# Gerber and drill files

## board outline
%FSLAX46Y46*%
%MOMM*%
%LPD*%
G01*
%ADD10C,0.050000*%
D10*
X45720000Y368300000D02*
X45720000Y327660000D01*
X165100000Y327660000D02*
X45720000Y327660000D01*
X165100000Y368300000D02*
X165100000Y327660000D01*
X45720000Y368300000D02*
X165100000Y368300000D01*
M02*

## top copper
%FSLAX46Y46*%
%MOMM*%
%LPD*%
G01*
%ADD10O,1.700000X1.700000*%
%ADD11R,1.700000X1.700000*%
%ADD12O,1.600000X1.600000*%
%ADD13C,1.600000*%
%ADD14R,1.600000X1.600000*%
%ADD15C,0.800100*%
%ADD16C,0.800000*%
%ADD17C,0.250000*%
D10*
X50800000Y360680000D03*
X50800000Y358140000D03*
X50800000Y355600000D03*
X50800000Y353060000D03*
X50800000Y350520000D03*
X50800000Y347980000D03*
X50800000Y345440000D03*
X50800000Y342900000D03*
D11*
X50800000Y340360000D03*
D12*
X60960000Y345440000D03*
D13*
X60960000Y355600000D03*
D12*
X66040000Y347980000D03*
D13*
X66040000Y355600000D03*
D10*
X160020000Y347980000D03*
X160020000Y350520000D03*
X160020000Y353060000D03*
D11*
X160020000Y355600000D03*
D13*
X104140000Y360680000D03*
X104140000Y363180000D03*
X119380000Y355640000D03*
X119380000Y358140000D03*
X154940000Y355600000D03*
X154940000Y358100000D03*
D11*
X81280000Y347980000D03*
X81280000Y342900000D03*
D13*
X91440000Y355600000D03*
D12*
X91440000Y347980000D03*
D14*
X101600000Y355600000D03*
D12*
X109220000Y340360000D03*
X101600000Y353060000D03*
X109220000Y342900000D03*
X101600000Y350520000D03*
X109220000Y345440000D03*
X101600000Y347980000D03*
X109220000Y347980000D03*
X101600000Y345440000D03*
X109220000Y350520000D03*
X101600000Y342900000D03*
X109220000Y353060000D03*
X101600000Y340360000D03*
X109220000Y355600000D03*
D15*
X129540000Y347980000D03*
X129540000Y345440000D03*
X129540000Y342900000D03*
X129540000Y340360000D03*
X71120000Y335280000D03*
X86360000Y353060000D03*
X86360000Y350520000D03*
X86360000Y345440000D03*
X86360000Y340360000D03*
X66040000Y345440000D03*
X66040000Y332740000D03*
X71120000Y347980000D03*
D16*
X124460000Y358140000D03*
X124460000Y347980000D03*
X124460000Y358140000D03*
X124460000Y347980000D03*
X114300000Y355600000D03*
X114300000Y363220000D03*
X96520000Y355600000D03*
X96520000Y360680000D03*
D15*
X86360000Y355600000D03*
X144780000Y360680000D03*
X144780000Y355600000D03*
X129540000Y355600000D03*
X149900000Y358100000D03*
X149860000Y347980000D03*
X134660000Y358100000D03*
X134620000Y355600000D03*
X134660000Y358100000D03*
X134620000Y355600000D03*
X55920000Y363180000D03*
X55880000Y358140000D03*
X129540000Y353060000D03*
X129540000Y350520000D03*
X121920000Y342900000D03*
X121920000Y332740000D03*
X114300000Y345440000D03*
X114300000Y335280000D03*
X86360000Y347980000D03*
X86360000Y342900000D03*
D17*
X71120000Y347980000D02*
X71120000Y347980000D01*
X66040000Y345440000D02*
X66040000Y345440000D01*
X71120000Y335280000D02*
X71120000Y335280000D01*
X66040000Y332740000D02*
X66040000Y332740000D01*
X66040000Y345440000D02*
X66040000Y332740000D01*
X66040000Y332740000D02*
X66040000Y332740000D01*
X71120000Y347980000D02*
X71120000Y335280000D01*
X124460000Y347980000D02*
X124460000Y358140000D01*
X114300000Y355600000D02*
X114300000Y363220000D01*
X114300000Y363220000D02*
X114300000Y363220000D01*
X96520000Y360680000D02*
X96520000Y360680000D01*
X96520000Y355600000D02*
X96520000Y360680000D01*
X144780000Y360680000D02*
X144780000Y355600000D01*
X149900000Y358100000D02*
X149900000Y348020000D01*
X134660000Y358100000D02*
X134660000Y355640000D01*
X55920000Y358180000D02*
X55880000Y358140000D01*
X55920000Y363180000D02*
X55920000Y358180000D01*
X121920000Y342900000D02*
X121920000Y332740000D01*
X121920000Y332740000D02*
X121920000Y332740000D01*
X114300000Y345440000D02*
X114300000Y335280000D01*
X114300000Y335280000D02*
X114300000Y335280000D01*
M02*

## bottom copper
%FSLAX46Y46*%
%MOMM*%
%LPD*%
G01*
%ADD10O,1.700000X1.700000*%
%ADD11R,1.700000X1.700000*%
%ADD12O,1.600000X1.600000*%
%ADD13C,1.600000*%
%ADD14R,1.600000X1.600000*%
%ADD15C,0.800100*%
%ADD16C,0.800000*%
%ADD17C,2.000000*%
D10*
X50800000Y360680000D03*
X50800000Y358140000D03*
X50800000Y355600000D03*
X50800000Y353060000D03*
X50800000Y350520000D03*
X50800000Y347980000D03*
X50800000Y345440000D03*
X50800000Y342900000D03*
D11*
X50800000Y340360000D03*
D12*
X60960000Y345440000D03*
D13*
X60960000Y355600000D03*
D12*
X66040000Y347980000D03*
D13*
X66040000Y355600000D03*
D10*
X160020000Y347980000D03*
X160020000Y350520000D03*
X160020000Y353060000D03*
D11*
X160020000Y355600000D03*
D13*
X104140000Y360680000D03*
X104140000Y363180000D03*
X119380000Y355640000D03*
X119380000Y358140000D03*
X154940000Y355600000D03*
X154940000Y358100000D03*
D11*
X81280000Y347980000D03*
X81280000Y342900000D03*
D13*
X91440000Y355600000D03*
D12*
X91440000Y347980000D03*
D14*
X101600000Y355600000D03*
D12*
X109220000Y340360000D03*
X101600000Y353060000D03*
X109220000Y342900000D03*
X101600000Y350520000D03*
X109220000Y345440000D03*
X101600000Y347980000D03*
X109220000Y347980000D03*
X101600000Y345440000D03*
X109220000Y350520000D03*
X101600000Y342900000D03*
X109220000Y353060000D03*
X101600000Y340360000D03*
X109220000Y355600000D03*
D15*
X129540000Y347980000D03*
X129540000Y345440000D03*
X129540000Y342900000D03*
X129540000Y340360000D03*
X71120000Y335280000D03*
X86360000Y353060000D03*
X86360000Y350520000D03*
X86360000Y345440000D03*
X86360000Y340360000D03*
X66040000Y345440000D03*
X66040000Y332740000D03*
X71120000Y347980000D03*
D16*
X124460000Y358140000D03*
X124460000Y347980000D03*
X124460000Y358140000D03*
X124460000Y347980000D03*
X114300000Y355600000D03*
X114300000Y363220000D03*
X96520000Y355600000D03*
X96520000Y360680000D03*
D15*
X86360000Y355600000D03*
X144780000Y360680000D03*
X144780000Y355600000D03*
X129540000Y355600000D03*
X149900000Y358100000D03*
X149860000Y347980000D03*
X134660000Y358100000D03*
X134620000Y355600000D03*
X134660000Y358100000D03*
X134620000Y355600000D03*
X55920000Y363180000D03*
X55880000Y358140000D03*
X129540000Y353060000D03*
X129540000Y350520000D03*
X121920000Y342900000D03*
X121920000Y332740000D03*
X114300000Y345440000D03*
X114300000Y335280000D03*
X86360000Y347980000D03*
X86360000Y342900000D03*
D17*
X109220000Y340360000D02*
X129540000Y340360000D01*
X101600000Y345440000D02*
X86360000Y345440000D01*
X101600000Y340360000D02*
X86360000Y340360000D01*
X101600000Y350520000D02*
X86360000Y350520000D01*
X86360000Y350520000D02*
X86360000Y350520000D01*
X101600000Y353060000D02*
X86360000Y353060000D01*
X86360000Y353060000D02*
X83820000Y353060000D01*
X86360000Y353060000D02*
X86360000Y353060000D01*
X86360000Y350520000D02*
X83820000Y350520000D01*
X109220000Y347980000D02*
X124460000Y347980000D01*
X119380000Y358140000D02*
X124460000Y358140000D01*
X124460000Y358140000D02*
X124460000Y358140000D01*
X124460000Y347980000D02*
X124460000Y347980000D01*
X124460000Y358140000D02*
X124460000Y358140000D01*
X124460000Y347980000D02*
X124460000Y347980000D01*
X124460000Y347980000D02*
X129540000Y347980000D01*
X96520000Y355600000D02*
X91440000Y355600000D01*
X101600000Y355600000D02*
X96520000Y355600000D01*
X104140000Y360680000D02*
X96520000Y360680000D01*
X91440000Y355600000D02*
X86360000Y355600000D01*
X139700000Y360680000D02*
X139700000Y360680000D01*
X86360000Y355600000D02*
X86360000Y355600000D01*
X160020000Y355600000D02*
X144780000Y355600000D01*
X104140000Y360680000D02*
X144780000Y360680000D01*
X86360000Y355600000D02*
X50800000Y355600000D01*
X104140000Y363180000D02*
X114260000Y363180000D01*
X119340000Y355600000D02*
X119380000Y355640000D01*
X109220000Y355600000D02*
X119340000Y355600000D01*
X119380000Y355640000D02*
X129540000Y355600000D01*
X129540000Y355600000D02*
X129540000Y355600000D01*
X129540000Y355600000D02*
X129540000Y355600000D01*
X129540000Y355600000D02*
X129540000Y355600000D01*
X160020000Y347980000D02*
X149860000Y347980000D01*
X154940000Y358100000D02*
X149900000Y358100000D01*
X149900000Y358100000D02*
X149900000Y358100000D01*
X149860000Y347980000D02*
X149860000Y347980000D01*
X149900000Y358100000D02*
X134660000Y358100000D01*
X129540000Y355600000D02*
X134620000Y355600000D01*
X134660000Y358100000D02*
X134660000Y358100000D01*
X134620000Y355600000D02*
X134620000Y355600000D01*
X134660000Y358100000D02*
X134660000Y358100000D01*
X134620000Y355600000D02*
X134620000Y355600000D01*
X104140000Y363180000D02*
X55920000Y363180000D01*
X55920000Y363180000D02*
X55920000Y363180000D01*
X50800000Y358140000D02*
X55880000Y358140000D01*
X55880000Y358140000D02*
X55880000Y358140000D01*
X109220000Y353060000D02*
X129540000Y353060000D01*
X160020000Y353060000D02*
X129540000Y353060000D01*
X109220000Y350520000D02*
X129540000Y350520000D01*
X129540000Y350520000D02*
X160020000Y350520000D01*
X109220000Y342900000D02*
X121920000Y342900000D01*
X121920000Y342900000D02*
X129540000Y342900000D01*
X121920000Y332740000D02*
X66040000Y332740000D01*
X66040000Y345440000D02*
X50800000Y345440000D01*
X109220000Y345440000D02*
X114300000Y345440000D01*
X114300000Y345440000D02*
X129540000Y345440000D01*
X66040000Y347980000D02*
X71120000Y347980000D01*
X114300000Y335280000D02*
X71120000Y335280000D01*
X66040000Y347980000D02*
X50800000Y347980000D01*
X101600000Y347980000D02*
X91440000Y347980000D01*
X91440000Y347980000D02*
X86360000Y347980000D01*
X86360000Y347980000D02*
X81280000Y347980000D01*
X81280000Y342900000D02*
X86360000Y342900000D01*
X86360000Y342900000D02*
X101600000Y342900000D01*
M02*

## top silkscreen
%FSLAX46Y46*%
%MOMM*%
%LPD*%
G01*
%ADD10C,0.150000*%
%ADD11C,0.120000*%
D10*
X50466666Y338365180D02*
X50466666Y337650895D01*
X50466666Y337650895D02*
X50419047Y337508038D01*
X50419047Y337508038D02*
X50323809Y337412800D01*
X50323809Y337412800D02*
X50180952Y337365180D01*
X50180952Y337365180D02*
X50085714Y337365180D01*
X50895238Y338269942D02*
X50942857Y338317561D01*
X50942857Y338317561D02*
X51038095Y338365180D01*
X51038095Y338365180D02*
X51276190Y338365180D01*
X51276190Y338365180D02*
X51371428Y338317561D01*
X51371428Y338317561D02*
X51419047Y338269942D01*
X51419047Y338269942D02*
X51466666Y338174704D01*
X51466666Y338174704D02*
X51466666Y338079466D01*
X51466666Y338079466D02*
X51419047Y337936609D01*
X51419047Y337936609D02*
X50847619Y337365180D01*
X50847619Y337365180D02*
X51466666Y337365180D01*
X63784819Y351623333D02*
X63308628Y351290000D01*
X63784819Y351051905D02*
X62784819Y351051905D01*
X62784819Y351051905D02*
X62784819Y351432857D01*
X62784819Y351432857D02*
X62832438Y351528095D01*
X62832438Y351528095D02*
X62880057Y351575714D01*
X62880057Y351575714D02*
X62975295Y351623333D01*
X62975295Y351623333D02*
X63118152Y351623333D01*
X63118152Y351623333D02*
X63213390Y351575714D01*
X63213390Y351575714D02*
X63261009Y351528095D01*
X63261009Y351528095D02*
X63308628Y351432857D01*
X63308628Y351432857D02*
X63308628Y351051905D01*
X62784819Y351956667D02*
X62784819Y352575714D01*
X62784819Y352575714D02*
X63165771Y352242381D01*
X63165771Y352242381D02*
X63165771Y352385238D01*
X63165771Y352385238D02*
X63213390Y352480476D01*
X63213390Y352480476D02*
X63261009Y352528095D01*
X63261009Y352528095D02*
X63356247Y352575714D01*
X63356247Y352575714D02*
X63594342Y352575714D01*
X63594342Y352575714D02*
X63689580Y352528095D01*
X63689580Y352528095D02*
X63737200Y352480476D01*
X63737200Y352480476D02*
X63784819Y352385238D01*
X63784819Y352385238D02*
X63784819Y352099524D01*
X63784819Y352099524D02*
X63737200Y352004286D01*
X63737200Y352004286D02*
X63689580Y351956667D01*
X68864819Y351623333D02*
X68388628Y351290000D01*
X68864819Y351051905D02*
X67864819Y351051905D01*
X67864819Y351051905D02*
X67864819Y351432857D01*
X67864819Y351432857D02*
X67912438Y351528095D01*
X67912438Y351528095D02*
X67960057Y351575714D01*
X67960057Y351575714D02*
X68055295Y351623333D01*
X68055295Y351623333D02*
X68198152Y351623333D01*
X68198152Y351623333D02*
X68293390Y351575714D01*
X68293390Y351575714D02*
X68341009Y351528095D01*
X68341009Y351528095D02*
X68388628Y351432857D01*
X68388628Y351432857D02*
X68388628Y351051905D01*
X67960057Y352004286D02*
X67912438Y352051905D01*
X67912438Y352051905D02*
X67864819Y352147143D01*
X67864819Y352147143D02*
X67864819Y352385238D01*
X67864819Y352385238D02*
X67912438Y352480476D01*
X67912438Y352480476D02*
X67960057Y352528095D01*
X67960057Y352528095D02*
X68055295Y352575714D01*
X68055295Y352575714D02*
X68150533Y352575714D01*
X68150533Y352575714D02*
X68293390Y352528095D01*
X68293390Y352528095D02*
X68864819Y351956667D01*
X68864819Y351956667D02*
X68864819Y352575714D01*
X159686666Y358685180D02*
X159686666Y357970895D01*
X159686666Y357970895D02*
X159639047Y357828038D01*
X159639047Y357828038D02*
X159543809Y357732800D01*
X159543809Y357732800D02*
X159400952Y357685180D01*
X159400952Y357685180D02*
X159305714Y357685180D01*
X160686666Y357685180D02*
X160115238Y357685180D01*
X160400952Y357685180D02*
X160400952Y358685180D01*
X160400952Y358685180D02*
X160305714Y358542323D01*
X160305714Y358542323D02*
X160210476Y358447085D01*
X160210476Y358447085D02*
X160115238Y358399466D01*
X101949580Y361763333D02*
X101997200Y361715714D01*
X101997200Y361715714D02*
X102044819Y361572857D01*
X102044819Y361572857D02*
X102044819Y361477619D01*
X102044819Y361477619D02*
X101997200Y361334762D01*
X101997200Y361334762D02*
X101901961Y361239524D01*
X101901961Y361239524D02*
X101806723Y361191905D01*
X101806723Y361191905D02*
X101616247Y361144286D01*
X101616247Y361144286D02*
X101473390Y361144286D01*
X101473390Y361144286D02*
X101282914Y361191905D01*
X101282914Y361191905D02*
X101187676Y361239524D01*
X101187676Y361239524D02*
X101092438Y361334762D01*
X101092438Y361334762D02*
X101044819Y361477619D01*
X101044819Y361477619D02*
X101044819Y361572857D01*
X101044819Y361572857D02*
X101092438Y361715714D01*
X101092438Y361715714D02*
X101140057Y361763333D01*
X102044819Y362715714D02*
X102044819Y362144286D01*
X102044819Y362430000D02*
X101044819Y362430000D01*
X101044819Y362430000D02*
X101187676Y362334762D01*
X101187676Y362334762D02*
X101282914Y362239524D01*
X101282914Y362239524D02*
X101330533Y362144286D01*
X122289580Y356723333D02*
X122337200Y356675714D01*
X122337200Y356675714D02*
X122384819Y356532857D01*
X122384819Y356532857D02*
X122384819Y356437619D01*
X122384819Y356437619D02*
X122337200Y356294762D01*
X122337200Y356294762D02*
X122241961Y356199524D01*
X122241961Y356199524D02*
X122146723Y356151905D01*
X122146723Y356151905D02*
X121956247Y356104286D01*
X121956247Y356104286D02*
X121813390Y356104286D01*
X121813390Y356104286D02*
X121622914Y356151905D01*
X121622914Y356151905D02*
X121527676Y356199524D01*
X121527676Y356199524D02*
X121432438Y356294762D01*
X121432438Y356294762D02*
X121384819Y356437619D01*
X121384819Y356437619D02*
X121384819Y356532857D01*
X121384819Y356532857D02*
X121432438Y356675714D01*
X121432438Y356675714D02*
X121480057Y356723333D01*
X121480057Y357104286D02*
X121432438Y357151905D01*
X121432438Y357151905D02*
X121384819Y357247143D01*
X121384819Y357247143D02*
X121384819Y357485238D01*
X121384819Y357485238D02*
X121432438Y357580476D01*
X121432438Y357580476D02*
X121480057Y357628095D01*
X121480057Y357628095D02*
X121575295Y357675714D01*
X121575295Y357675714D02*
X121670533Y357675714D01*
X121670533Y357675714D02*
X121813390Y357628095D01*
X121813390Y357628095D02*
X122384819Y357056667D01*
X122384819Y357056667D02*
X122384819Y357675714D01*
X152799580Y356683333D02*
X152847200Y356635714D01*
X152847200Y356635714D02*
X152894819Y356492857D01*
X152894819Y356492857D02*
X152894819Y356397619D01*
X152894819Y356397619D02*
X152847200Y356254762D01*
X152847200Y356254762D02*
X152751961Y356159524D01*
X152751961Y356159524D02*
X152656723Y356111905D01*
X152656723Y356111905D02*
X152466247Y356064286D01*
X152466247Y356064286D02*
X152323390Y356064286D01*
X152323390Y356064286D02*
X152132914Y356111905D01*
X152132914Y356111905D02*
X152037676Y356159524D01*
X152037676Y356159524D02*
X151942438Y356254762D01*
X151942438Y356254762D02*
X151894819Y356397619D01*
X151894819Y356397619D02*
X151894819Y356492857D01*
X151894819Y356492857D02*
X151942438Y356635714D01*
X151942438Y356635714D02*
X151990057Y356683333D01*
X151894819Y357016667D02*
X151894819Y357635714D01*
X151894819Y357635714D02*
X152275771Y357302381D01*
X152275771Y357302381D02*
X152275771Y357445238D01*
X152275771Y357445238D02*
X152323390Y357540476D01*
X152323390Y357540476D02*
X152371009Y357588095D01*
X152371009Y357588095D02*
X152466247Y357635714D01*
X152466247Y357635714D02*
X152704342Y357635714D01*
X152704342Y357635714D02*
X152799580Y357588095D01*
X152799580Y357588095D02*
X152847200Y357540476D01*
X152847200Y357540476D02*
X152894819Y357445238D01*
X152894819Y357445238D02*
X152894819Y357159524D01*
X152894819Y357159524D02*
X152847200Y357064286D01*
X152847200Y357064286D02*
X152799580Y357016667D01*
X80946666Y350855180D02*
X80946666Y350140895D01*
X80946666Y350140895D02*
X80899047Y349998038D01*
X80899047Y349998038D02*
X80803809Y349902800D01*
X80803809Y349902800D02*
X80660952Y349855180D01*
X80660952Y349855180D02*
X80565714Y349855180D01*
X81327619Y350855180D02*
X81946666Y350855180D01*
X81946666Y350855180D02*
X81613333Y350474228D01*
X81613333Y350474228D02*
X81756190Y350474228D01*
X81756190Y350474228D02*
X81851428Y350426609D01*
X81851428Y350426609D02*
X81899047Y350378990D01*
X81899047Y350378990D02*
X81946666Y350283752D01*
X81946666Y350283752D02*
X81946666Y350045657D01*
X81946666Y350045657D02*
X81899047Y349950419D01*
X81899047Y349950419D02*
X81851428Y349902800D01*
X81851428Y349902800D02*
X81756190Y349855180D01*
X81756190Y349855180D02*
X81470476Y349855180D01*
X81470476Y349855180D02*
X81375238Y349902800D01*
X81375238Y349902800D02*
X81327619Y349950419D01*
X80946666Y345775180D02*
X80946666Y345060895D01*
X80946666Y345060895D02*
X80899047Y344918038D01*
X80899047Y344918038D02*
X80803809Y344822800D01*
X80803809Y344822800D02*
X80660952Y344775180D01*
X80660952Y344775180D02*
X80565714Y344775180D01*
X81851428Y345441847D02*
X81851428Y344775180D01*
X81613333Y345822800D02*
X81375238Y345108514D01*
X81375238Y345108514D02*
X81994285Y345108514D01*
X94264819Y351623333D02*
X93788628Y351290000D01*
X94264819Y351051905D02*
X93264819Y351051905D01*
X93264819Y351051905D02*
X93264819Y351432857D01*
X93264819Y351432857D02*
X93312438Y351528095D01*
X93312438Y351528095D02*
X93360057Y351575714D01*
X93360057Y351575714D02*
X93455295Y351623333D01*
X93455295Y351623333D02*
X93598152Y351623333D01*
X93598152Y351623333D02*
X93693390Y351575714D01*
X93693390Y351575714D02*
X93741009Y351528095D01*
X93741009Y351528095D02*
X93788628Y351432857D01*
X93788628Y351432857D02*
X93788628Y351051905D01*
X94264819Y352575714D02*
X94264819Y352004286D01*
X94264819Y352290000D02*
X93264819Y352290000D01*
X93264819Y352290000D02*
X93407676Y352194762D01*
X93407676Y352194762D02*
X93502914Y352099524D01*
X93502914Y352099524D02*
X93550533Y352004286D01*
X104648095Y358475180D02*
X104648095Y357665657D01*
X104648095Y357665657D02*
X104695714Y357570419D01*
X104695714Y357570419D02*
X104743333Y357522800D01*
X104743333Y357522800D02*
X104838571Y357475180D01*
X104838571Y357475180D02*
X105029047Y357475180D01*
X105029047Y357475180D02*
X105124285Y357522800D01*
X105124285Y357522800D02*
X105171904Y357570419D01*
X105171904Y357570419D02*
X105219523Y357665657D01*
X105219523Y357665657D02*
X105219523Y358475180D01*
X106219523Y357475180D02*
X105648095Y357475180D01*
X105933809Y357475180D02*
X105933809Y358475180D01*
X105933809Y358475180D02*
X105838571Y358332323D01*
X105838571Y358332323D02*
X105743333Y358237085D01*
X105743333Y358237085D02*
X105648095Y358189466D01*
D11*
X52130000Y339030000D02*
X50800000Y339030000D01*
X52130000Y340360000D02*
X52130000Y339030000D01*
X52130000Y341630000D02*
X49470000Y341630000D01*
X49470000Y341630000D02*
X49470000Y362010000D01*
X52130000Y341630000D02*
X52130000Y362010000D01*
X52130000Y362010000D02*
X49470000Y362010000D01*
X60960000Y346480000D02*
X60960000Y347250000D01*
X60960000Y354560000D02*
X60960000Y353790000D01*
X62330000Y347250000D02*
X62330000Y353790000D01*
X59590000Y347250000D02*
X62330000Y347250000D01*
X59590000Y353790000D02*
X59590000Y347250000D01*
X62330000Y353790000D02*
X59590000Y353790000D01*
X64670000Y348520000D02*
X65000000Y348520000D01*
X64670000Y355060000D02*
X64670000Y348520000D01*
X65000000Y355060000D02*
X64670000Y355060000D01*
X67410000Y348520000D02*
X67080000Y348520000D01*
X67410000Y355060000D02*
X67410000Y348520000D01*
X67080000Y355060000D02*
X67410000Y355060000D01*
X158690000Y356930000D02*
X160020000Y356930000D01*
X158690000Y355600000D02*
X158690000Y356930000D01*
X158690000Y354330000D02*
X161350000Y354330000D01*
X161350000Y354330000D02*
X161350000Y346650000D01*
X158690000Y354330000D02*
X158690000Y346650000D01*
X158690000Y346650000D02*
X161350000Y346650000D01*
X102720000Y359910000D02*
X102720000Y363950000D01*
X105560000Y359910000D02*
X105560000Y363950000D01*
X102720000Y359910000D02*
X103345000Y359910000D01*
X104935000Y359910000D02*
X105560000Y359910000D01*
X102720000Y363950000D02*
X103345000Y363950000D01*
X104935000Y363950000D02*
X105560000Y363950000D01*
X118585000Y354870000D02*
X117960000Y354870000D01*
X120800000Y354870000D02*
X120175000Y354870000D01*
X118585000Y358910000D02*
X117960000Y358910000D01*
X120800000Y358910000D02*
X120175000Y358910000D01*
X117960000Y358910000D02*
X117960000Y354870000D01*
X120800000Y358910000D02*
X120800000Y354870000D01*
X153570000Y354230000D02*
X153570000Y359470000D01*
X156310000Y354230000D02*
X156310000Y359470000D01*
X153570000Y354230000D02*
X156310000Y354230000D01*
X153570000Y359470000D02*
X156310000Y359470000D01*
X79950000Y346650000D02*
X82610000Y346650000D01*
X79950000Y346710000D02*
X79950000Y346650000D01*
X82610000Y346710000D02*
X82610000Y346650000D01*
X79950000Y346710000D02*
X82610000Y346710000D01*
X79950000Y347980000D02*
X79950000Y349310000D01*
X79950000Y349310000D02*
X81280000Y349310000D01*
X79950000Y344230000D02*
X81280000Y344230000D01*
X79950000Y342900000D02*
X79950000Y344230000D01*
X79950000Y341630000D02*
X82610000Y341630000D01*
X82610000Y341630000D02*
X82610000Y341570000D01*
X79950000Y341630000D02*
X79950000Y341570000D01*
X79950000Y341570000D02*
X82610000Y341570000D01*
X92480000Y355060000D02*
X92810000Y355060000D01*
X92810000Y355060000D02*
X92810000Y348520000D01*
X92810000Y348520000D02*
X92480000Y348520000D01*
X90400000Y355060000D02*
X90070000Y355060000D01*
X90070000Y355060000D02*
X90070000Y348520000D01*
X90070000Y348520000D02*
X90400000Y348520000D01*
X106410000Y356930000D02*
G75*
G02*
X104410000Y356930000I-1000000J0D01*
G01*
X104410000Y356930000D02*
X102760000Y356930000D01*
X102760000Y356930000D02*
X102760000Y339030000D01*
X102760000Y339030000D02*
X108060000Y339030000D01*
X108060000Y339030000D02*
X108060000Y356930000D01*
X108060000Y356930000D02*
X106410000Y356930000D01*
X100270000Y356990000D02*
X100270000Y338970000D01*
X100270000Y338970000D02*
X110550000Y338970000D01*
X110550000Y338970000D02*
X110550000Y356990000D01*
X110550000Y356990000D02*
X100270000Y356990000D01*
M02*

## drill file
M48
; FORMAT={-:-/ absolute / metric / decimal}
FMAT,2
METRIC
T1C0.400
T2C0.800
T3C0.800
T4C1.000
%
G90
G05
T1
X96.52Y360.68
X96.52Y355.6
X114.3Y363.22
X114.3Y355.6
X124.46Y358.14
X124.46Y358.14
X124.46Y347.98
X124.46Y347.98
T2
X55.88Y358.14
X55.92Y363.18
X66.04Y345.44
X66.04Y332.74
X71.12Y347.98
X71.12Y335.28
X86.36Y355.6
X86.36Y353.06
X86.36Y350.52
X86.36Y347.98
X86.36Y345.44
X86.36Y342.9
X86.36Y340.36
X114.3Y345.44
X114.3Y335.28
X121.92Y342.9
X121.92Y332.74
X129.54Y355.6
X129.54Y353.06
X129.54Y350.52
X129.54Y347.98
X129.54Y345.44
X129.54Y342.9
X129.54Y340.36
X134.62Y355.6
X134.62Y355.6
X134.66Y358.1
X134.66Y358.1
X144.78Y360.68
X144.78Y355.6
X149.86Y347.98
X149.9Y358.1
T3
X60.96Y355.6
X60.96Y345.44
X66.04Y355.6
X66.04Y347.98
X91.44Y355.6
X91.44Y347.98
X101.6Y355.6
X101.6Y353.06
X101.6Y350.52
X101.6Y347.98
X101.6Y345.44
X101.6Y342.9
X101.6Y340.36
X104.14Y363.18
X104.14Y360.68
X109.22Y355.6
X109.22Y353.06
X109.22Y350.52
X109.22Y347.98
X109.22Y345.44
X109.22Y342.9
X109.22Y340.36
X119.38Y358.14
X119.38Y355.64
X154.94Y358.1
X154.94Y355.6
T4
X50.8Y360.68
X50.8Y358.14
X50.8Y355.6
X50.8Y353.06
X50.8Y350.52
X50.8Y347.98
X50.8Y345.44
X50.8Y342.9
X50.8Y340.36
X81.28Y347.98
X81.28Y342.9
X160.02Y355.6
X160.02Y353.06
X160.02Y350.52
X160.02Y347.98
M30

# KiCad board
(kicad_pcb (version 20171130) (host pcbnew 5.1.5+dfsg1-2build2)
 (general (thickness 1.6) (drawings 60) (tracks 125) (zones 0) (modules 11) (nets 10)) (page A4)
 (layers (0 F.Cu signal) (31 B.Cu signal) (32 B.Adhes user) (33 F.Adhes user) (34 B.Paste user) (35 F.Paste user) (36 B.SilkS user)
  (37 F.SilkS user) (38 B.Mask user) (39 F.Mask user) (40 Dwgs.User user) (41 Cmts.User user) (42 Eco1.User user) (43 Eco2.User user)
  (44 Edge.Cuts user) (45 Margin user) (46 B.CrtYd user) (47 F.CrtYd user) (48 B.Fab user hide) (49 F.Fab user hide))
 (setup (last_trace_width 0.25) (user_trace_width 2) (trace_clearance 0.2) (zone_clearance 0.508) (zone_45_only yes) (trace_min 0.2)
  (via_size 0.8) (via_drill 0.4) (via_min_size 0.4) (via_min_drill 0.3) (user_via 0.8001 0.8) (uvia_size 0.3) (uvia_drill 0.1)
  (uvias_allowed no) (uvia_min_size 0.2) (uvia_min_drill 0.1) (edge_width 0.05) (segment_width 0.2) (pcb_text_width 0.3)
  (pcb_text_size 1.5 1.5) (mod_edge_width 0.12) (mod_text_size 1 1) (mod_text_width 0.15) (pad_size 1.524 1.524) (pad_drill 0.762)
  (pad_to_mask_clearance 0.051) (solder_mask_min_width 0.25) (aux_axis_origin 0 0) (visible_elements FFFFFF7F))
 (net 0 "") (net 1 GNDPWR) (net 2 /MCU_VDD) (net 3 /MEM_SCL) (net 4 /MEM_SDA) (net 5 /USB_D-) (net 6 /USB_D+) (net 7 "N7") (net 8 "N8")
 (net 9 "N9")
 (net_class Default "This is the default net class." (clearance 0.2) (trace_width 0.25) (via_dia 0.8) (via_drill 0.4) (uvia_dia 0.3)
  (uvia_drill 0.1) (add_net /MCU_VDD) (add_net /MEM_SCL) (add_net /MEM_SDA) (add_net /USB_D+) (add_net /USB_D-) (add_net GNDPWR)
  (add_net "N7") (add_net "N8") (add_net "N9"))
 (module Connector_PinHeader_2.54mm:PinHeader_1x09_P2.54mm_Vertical (layer F.Cu) (at 50.8 -340.36 180)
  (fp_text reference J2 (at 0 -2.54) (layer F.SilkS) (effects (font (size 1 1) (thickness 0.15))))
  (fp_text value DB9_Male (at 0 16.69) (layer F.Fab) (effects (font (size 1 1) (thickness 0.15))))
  (fp_line (start -1.33 -1.33) (end 0 -1.33) (layer F.SilkS) (width 0.12))
  (fp_line (start -1.33 0) (end -1.33 -1.33) (layer F.SilkS) (width 0.12))
  (fp_line (start -1.33 1.27) (end 1.33 1.27) (layer F.SilkS) (width 0.12))
  (fp_line (start 1.33 1.27) (end 1.33 21.65) (layer F.SilkS) (width 0.12))
  (fp_line (start -1.33 1.27) (end -1.33 21.65) (layer F.SilkS) (width 0.12))
  (fp_line (start -1.33 21.65) (end 1.33 21.65) (layer F.SilkS) (width 0.12))
  (pad 9 thru_hole oval (at 0 20.32 180) (size 1.7 1.7) (drill 1) (layers *.Cu *.Mask))
  (pad 8 thru_hole oval (at 0 17.78 180) (size 1.7 1.7) (drill 1) (layers *.Cu *.Mask) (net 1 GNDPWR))
  (pad 7 thru_hole oval (at 0 15.24 180) (size 1.7 1.7) (drill 1) (layers *.Cu *.Mask) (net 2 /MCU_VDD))
  (pad 6 thru_hole oval (at 0 12.7 180) (size 1.7 1.7) (drill 1) (layers *.Cu *.Mask))
  (pad 5 thru_hole oval (at 0 10.16 180) (size 1.7 1.7) (drill 1) (layers *.Cu *.Mask))
  (pad 4 thru_hole oval (at 0 7.62 180) (size 1.7 1.7) (drill 1) (layers *.Cu *.Mask) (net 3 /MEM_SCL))
  (pad 3 thru_hole oval (at 0 5.08 180) (size 1.7 1.7) (drill 1) (layers *.Cu *.Mask) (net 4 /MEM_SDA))
  (pad 2 thru_hole oval (at 0 2.54 180) (size 1.7 1.7) (drill 1) (layers *.Cu *.Mask))
  (pad 1 thru_hole rect (at 0 0 180) (size 1.7 1.7) (drill 1) (layers *.Cu *.Mask)))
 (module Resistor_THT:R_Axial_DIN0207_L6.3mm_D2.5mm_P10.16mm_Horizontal (layer F.Cu) (at 60.96 -355.6 270)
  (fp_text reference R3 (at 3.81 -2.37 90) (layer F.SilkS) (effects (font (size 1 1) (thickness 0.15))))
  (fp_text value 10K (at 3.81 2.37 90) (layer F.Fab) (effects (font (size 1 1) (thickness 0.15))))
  (fp_line (start 9.12 0) (end 8.35 0) (layer F.SilkS) (width 0.12))
  (fp_line (start 1.04 0) (end 1.81 0) (layer F.SilkS) (width 0.12))
  (fp_line (start 8.35 -1.37) (end 1.81 -1.37) (layer F.SilkS) (width 0.12))
  (fp_line (start 8.35 1.37) (end 8.35 -1.37) (layer F.SilkS) (width 0.12))
  (fp_line (start 1.81 1.37) (end 8.35 1.37) (layer F.SilkS) (width 0.12))
  (fp_line (start 1.81 -1.37) (end 1.81 1.37) (layer F.SilkS) (width 0.12))
  (pad 2 thru_hole oval (at 10.16 0 270) (size 1.6 1.6) (drill 0.8) (layers *.Cu *.Mask) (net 4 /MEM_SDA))
  (pad 1 thru_hole circle (at 0 0 270) (size 1.6 1.6) (drill 0.8) (layers *.Cu *.Mask) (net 2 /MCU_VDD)))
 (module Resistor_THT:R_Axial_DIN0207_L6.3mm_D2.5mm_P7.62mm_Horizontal (layer F.Cu) (at 66.04 -355.6 270)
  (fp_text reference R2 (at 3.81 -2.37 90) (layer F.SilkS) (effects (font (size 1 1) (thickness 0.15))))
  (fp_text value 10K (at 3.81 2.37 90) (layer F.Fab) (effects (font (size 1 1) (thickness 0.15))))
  (fp_line (start 7.08 1.37) (end 7.08 1.04) (layer F.SilkS) (width 0.12))
  (fp_line (start 0.54 1.37) (end 7.08 1.37) (layer F.SilkS) (width 0.12))
  (fp_line (start 0.54 1.04) (end 0.54 1.37) (layer F.SilkS) (width 0.12))
  (fp_line (start 7.08 -1.37) (end 7.08 -1.04) (layer F.SilkS) (width 0.12))
  (fp_line (start 0.54 -1.37) (end 7.08 -1.37) (layer F.SilkS) (width 0.12))
  (fp_line (start 0.54 -1.04) (end 0.54 -1.37) (layer F.SilkS) (width 0.12))
  (pad 2 thru_hole oval (at 7.62 0 270) (size 1.6 1.6) (drill 0.8) (layers *.Cu *.Mask) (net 3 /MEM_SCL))
  (pad 1 thru_hole circle (at 0 0 270) (size 1.6 1.6) (drill 0.8) (layers *.Cu *.Mask) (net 2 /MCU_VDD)))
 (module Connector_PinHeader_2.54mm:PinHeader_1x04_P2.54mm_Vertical (layer F.Cu) (at 160.02 -355.6)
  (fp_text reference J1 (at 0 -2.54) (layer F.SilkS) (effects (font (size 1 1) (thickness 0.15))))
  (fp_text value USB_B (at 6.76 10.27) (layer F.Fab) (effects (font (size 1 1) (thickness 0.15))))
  (fp_line (start -1.33 -1.33) (end 0 -1.33) (layer F.SilkS) (width 0.12))
  (fp_line (start -1.33 0) (end -1.33 -1.33) (layer F.SilkS) (width 0.12))
  (fp_line (start -1.33 1.27) (end 1.33 1.27) (layer F.SilkS) (width 0.12))
  (fp_line (start 1.33 1.27) (end 1.33 8.95) (layer F.SilkS) (width 0.12))
  (fp_line (start -1.33 1.27) (end -1.33 8.95) (layer F.SilkS) (width 0.12))
  (fp_line (start -1.33 8.95) (end 1.33 8.95) (layer F.SilkS) (width 0.12))
  (pad 4 thru_hole oval (at 0 7.62) (size 1.7 1.7) (drill 1) (layers *.Cu *.Mask) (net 1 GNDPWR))
  (pad 3 thru_hole oval (at 0 5.08) (size 1.7 1.7) (drill 1) (layers *.Cu *.Mask) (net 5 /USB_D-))
  (pad 2 thru_hole oval (at 0 2.54) (size 1.7 1.7) (drill 1) (layers *.Cu *.Mask) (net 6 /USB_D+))
  (pad 1 thru_hole rect (at 0 0) (size 1.7 1.7) (drill 1) (layers *.Cu *.Mask) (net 2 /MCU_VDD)))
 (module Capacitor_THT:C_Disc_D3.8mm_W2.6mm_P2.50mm (layer F.Cu) (at 104.14 -360.68 90)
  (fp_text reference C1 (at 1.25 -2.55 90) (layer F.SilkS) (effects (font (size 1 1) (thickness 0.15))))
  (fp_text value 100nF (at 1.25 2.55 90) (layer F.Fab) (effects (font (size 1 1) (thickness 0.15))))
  (fp_line (start -0.77 -1.42) (end 3.27 -1.42) (layer F.SilkS) (width 0.12))
  (fp_line (start -0.77 1.42) (end 3.27 1.42) (layer F.SilkS) (width 0.12))
  (fp_line (start -0.77 -1.42) (end -0.77 -0.795) (layer F.SilkS) (width 0.12))
  (fp_line (start -0.77 0.795) (end -0.77 1.42) (layer F.SilkS) (width 0.12))
  (fp_line (start 3.27 -1.42) (end 3.27 -0.795) (layer F.SilkS) (width 0.12))
  (fp_line (start 3.27 0.795) (end 3.27 1.42) (layer F.SilkS) (width 0.12))
  (pad 1 thru_hole circle (at 0 0 90) (size 1.6 1.6) (drill 0.8) (layers *.Cu *.Mask) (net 2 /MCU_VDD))
  (pad 2 thru_hole circle (at 2.5 0 90) (size 1.6 1.6) (drill 0.8) (layers *.Cu *.Mask) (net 1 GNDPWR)))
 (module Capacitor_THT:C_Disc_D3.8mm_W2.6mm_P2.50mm (layer F.Cu) (at 119.38 -358.14 270)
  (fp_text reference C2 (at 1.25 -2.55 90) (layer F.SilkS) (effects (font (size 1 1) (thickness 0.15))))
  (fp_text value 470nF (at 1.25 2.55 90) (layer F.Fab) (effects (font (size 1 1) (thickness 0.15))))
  (fp_line (start 3.27 0.795) (end 3.27 1.42) (layer F.SilkS) (width 0.12))
  (fp_line (start 3.27 -1.42) (end 3.27 -0.795) (layer F.SilkS) (width 0.12))
  (fp_line (start -0.77 0.795) (end -0.77 1.42) (layer F.SilkS) (width 0.12))
  (fp_line (start -0.77 -1.42) (end -0.77 -0.795) (layer F.SilkS) (width 0.12))
  (fp_line (start -0.77 1.42) (end 3.27 1.42) (layer F.SilkS) (width 0.12))
  (fp_line (start -0.77 -1.42) (end 3.27 -1.42) (layer F.SilkS) (width 0.12))
  (pad 2 thru_hole circle (at 2.5 0 270) (size 1.6 1.6) (drill 0.8) (layers *.Cu *.Mask) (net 1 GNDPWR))
  (pad 1 thru_hole circle (at 0 0 270) (size 1.6 1.6) (drill 0.8) (layers *.Cu *.Mask) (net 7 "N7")))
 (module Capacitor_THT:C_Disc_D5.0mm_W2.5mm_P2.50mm (layer F.Cu) (at 154.94 -355.6 90)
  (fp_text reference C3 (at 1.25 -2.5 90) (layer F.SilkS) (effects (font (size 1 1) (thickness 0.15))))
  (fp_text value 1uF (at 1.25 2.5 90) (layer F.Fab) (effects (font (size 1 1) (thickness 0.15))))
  (fp_line (start -1.37 -1.37) (end 3.87 -1.37) (layer F.SilkS) (width 0.12))
  (fp_line (start -1.37 1.37) (end 3.87 1.37) (layer F.SilkS) (width 0.12))
  (fp_line (start -1.37 -1.37) (end -1.37 1.37) (layer F.SilkS) (width 0.12))
  (fp_line (start 3.87 -1.37) (end 3.87 1.37) (layer F.SilkS) (width 0.12))
  (pad 1 thru_hole circle (at 0 0 90) (size 1.6 1.6) (drill 0.8) (layers *.Cu *.Mask) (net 2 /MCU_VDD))
  (pad 2 thru_hole circle (at 2.5 0 90) (size 1.6 1.6) (drill 0.8) (layers *.Cu *.Mask) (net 1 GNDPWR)))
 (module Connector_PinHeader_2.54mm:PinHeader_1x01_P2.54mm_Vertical (layer F.Cu) (at 81.28 -347.98)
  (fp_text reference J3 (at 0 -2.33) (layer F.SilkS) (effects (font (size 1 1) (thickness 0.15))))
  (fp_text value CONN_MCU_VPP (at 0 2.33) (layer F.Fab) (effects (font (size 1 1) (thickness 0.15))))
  (fp_line (start -1.33 1.33) (end 1.33 1.33) (layer F.SilkS) (width 0.12))
  (fp_line (start -1.33 1.27) (end -1.33 1.33) (layer F.SilkS) (width 0.12))
  (fp_line (start 1.33 1.27) (end 1.33 1.33) (layer F.SilkS) (width 0.12))
  (fp_line (start -1.33 1.27) (end 1.33 1.27) (layer F.SilkS) (width 0.12))
  (fp_line (start -1.33 0) (end -1.33 -1.33) (layer F.SilkS) (width 0.12))
  (fp_line (start -1.33 -1.33) (end 0 -1.33) (layer F.SilkS) (width 0.12))
  (pad 1 thru_hole rect (at 0 0) (size 1.7 1.7) (drill 1) (layers *.Cu *.Mask) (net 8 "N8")))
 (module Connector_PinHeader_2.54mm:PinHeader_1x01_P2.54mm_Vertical (layer F.Cu) (at 81.28 -342.9)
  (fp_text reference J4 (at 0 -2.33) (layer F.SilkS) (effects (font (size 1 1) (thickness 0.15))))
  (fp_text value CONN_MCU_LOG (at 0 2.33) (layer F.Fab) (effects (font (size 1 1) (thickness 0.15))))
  (fp_line (start -1.33 -1.33) (end 0 -1.33) (layer F.SilkS) (width 0.12))
  (fp_line (start -1.33 0) (end -1.33 -1.33) (layer F.SilkS) (width 0.12))
  (fp_line (start -1.33 1.27) (end 1.33 1.27) (layer F.SilkS) (width 0.12))
  (fp_line (start 1.33 1.27) (end 1.33 1.33) (layer F.SilkS) (width 0.12))
  (fp_line (start -1.33 1.27) (end -1.33 1.33) (layer F.SilkS) (width 0.12))
  (fp_line (start -1.33 1.33) (end 1.33 1.33) (layer F.SilkS) (width 0.12))
  (pad 1 thru_hole rect (at 0 0) (size 1.7 1.7) (drill 1) (layers *.Cu *.Mask) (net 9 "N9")))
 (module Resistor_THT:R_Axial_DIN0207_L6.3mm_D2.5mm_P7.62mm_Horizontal (layer F.Cu) (at 91.44 -355.6 270)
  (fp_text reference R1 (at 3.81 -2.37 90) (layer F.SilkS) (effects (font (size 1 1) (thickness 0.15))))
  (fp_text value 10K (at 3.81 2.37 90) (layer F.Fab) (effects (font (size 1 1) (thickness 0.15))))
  (fp_line (start 0.54 -1.04) (end 0.54 -1.37) (layer F.SilkS) (width 0.12))
  (fp_line (start 0.54 -1.37) (end 7.08 -1.37) (layer F.SilkS) (width 0.12))
  (fp_line (start 7.08 -1.37) (end 7.08 -1.04) (layer F.SilkS) (width 0.12))
  (fp_line (start 0.54 1.04) (end 0.54 1.37) (layer F.SilkS) (width 0.12))
  (fp_line (start 0.54 1.37) (end 7.08 1.37) (layer F.SilkS) (width 0.12))
  (fp_line (start 7.08 1.37) (end 7.08 1.04) (layer F.SilkS) (width 0.12))
  (pad 1 thru_hole circle (at 0 0 270) (size 1.6 1.6) (drill 0.8) (layers *.Cu *.Mask) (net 2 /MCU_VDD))
  (pad 2 thru_hole oval (at 7.62 0 270) (size 1.6 1.6) (drill 0.8) (layers *.Cu *.Mask) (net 8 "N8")))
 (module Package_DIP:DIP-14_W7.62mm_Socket (layer F.Cu) (at 101.6 -355.6)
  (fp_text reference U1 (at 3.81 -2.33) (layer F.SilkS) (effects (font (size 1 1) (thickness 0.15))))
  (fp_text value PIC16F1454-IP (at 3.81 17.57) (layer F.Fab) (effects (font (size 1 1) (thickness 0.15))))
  (fp_arc (start 3.81 -1.33) (end 2.81 -1.33) (angle -180) (layer F.SilkS) (width 0.12))
  (fp_line (start 2.81 -1.33) (end 1.16 -1.33) (layer F.SilkS) (width 0.12))
  (fp_line (start 1.16 -1.33) (end 1.16 16.57) (layer F.SilkS) (width 0.12))
  (fp_line (start 1.16 16.57) (end 6.46 16.57) (layer F.SilkS) (width 0.12))
  (fp_line (start 6.46 16.57) (end 6.46 -1.33) (layer F.SilkS) (width 0.12))
  (fp_line (start 6.46 -1.33) (end 4.81 -1.33) (layer F.SilkS) (width 0.12))
  (fp_line (start -1.33 -1.39) (end -1.33 16.63) (layer F.SilkS) (width 0.12))
  (fp_line (start -1.33 16.63) (end 8.95 16.63) (layer F.SilkS) (width 0.12))
  (fp_line (start 8.95 16.63) (end 8.95 -1.39) (layer F.SilkS) (width 0.12))
  (fp_line (start 8.95 -1.39) (end -1.33 -1.39) (layer F.SilkS) (width 0.12))
  (pad 1 thru_hole rect (at 0 0) (size 1.6 1.6) (drill 0.8) (layers *.Cu *.Mask) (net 2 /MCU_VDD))
  (pad 8 thru_hole oval (at 7.62 15.24) (size 1.6 1.6) (drill 0.8) (layers *.Cu *.Mask))
  (pad 2 thru_hole oval (at 0 2.54) (size 1.6 1.6) (drill 0.8) (layers *.Cu *.Mask))
  (pad 9 thru_hole oval (at 7.62 12.7) (size 1.6 1.6) (drill 0.8) (layers *.Cu *.Mask) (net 4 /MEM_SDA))
  (pad 3 thru_hole oval (at 0 5.08) (size 1.6 1.6) (drill 0.8) (layers *.Cu *.Mask))
  (pad 10 thru_hole oval (at 7.62 10.16) (size 1.6 1.6) (drill 0.8) (layers *.Cu *.Mask) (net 3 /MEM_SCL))
  (pad 4 thru_hole oval (at 0 7.62) (size 1.6 1.6) (drill 0.8) (layers *.Cu *.Mask) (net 8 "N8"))
  (pad 11 thru_hole oval (at 7.62 7.62) (size 1.6 1.6) (drill 0.8) (layers *.Cu *.Mask) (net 7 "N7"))
  (pad 5 thru_hole oval (at 0 10.16) (size 1.6 1.6) (drill 0.8) (layers *.Cu *.Mask))
  (pad 12 thru_hole oval (at 7.62 5.08) (size 1.6 1.6) (drill 0.8) (layers *.Cu *.Mask) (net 5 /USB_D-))
  (pad 6 thru_hole oval (at 0 12.7) (size 1.6 1.6) (drill 0.8) (layers *.Cu *.Mask) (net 9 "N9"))
  (pad 13 thru_hole oval (at 7.62 2.54) (size 1.6 1.6) (drill 0.8) (layers *.Cu *.Mask) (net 6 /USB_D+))
  (pad 7 thru_hole oval (at 0 15.24) (size 1.6 1.6) (drill 0.8) (layers *.Cu *.Mask))
  (pad 14 thru_hole oval (at 7.62 0) (size 1.6 1.6) (drill 0.8) (layers *.Cu *.Mask) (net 1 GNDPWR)))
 (gr_line (start 45.72 -368.3) (end 45.72 -327.66) (layer Edge.Cuts) (width 0.05))
 (gr_line (start 165.1 -327.66) (end 45.72 -327.66) (layer Edge.Cuts) (width 0.05))
 (gr_line (start 165.1 -368.3) (end 165.1 -327.66) (layer Edge.Cuts) (width 0.05))
 (gr_line (start 45.72 -368.3) (end 165.1 -368.3) (layer Edge.Cuts) (width 0.05))
 (via (at 129.54 -347.98) (size 0.8001) (drill 0.8) (layers F.Cu B.Cu) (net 7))
 (via (at 129.54 -345.44) (size 0.8001) (drill 0.8) (layers F.Cu B.Cu) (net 3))
 (via (at 129.54 -342.9) (size 0.8001) (drill 0.8) (layers F.Cu B.Cu) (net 4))
 (via (at 129.54 -340.36) (size 0.8001) (drill 0.8) (layers F.Cu B.Cu) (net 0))
 (segment (start 109.22 -340.36) (end 129.54 -340.36) (width 2) (layer B.Cu) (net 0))
 (segment (start 101.6 -345.44) (end 86.36 -345.44) (width 2) (layer B.Cu) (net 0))
 (segment (start 101.6 -340.36) (end 86.36 -340.36) (width 2) (layer B.Cu) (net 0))
 (segment (start 101.6 -350.52) (end 86.36 -350.52) (width 2) (layer B.Cu) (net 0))
 (segment (start 86.36 -350.52) (end 86.36 -350.52) (width 2) (layer B.Cu) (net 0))
 (segment (start 101.6 -353.06) (end 86.36 -353.06) (width 2) (layer B.Cu) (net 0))
 (segment (start 86.36 -353.06) (end 83.82 -353.06) (width 2) (layer B.Cu) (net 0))
 (segment (start 71.12 -347.98) (end 71.12 -347.98) (width 0.25) (layer F.Cu) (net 3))
 (segment (start 66.04 -345.44) (end 66.04 -345.44) (width 0.25) (layer F.Cu) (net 4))
 (segment (start 71.12 -335.28) (end 71.12 -335.28) (width 0.25) (layer F.Cu) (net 3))
 (via (at 71.12 -335.28) (size 0.8001) (drill 0.8) (layers F.Cu B.Cu) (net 3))
 (segment (start 66.04 -332.74) (end 66.04 -332.74) (width 0.25) (layer F.Cu) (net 4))
 (segment (start 86.36 -353.06) (end 86.36 -353.06) (width 2) (layer B.Cu) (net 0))
 (via (at 86.36 -353.06) (size 0.8001) (drill 0.8) (layers F.Cu B.Cu) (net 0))
 (segment (start 86.36 -350.52) (end 83.82 -350.52) (width 2) (layer B.Cu) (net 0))
 (via (at 86.36 -350.52) (size 0.8001) (drill 0.8) (layers F.Cu B.Cu) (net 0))
 (via (at 86.36 -345.44) (size 0.8001) (drill 0.8) (layers F.Cu B.Cu) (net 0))
 (via (at 86.36 -340.36) (size 0.8001) (drill 0.8) (layers F.Cu B.Cu) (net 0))
 (segment (start 66.04 -345.44) (end 66.04 -332.74) (width 0.25) (layer F.Cu) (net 4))
 (via (at 66.04 -345.44) (size 0.8001) (drill 0.8) (layers F.Cu B.Cu) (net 4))
 (segment (start 66.04 -332.74) (end 66.04 -332.74) (width 0.25) (layer F.Cu) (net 4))
 (via (at 66.04 -332.74) (size 0.8001) (drill 0.8) (layers F.Cu B.Cu) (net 4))
 (segment (start 71.12 -347.98) (end 71.12 -335.28) (width 0.25) (layer F.Cu) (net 3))
 (via (at 71.12 -347.98) (size 0.8001) (drill 0.8) (layers F.Cu B.Cu) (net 3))
 (segment (start 109.22 -347.98) (end 124.46 -347.98) (width 2) (layer B.Cu) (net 7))
 (segment (start 119.38 -358.14) (end 124.46 -358.14) (width 2) (layer B.Cu) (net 7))
 (segment (start 124.46 -358.14) (end 124.46 -358.14) (width 2) (layer B.Cu) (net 7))
 (via (at 124.46 -358.14) (size 0.8) (drill 0.4) (layers F.Cu B.Cu) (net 7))
 (segment (start 124.46 -347.98) (end 124.46 -347.98) (width 2) (layer B.Cu) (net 7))
 (via (at 124.46 -347.98) (size 0.8) (drill 0.4) (layers F.Cu B.Cu) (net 7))
 (segment (start 124.46 -358.14) (end 124.46 -358.14) (width 2) (layer B.Cu) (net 7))
 (via (at 124.46 -358.14) (size 0.8) (drill 0.4) (layers F.Cu B.Cu) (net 7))
 (segment (start 124.46 -347.98) (end 124.46 -347.98) (width 2) (layer B.Cu) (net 7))
 (via (at 124.46 -347.98) (size 0.8) (drill 0.4) (layers F.Cu B.Cu) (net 7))
 (segment (start 124.46 -347.98) (end 124.46 -358.14) (width 0.25) (layer F.Cu) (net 7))
 (segment (start 124.46 -347.98) (end 129.54 -347.98) (width 2) (layer B.Cu) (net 7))
 (via (at 114.3 -355.6) (size 0.8) (drill 0.4) (layers F.Cu B.Cu) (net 1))
 (segment (start 114.3 -355.6) (end 114.3 -363.22) (width 0.25) (layer F.Cu) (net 1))
 (segment (start 114.3 -363.22) (end 114.3 -363.22) (width 0.25) (layer F.Cu) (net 1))
 (via (at 114.3 -363.22) (size 0.8) (drill 0.4) (layers F.Cu B.Cu) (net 1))
 (segment (start 96.52 -360.68) (end 96.52 -360.68) (width 0.25) (layer F.Cu) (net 2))
 (via (at 96.52 -355.6) (size 0.8) (drill 0.4) (layers F.Cu B.Cu) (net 2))
 (segment (start 96.52 -355.6) (end 91.44 -355.6) (width 2) (layer B.Cu) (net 2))
 (segment (start 101.6 -355.6) (end 96.52 -355.6) (width 2) (layer B.Cu) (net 2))
 (via (at 96.52 -360.68) (size 0.8) (drill 0.4) (layers F.Cu B.Cu) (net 2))
 (segment (start 96.52 -355.6) (end 96.52 -360.68) (width 0.25) (layer F.Cu) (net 2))
 (segment (start 104.14 -360.68) (end 96.52 -360.68) (width 2) (layer B.Cu) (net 2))
 (segment (start 91.44 -355.6) (end 86.36 -355.6) (width 2) (layer B.Cu) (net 2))
 (segment (start 139.7 -360.68) (end 139.7 -360.68) (width 2) (layer B.Cu) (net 2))
 (segment (start 86.36 -355.6) (end 86.36 -355.6) (width 2) (layer B.Cu) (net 2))
 (via (at 86.36 -355.6) (size 0.8001) (drill 0.8) (layers F.Cu B.Cu) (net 2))
 (segment (start 160.02 -355.6) (end 144.78 -355.6) (width 2) (layer B.Cu) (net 2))
 (segment (start 104.14 -360.68) (end 144.78 -360.68) (width 2) (layer B.Cu) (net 2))
 (via (at 144.78 -360.68) (size 0.8001) (drill 0.8) (layers F.Cu B.Cu) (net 2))
 (segment (start 144.78 -360.68) (end 144.78 -355.6) (width 0.25) (layer F.Cu) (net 2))
 (via (at 144.78 -355.6) (size 0.8001) (drill 0.8) (layers F.Cu B.Cu) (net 2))
 (segment (start 86.36 -355.6) (end 50.8 -355.6) (width 2) (layer B.Cu) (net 2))
 (segment (start 104.14 -363.18) (end 114.26 -363.18) (width 2) (layer B.Cu) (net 1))
 (segment (start 119.34 -355.6) (end 119.38 -355.64) (width 2) (layer B.Cu) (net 1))
 (segment (start 109.22 -355.6) (end 119.34 -355.6) (width 2) (layer B.Cu) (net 1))
 (segment (start 119.38 -355.64) (end 129.54 -355.6) (width 2) (layer B.Cu) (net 1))
 (segment (start 129.54 -355.6) (end 129.54 -355.6) (width 2) (layer B.Cu) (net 1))
 (segment (start 129.54 -355.6) (end 129.54 -355.6) (width 2) (layer B.Cu) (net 1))
 (segment (start 129.54 -355.6) (end 129.54 -355.6) (width 2) (layer B.Cu) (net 1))
 (via (at 129.54 -355.6) (size 0.8001) (drill 0.8) (layers F.Cu B.Cu) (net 1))
 (segment (start 160.02 -347.98) (end 149.86 -347.98) (width 2) (layer B.Cu) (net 1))
 (segment (start 154.94 -358.1) (end 149.9 -358.1) (width 2) (layer B.Cu) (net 1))
 (segment (start 149.9 -358.1) (end 149.9 -358.1) (width 2) (layer B.Cu) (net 1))
 (via (at 149.9 -358.1) (size 0.8001) (drill 0.8) (layers F.Cu B.Cu) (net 1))
 (segment (start 149.86 -347.98) (end 149.86 -347.98) (width 2) (layer B.Cu) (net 1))
 (via (at 149.86 -347.98) (size 0.8001) (drill 0.8) (layers F.Cu B.Cu) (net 1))
 (segment (start 149.9 -358.1) (end 149.9 -348.02) (width 0.25) (layer F.Cu) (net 1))
 (segment (start 149.9 -358.1) (end 134.66 -358.1) (width 2) (layer B.Cu) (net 1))
 (segment (start 129.54 -355.6) (end 134.62 -355.6) (width 2) (layer B.Cu) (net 1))
 (segment (start 134.66 -358.1) (end 134.66 -358.1) (width 2) (layer B.Cu) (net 1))
 (via (at 134.66 -358.1) (size 0.8001) (drill 0.8) (layers F.Cu B.Cu) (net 1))
 (segment (start 134.62 -355.6) (end 134.62 -355.6) (width 2) (layer B.Cu) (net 1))
 (via (at 134.62 -355.6) (size 0.8001) (drill 0.8) (layers F.Cu B.Cu) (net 1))
 (segment (start 134.66 -358.1) (end 134.66 -358.1) (width 2) (layer B.Cu) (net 1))
 (via (at 134.66 -358.1) (size 0.8001) (drill 0.8) (layers F.Cu B.Cu) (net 1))
 (segment (start 134.62 -355.6) (end 134.62 -355.6) (width 2) (layer B.Cu) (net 1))
 (via (at 134.62 -355.6) (size 0.8001) (drill 0.8) (layers F.Cu B.Cu) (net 1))
 (segment (start 134.66 -358.1) (end 134.66 -355.64) (width 0.25) (layer F.Cu) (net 1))
 (segment (start 104.14 -363.18) (end 55.92 -363.18) (width 2) (layer B.Cu) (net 1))
 (segment (start 55.92 -363.18) (end 55.92 -363.18) (width 2) (layer B.Cu) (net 1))
 (via (at 55.92 -363.18) (size 0.8001) (drill 0.8) (layers F.Cu B.Cu) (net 1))
 (segment (start 50.8 -358.14) (end 55.88 -358.14) (width 2) (layer B.Cu) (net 1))
 (segment (start 55.88 -358.14) (end 55.88 -358.14) (width 2) (layer B.Cu) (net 1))
 (via (at 55.88 -358.14) (size 0.8001) (drill 0.8) (layers F.Cu B.Cu) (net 1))
 (segment (start 55.92 -358.18) (end 55.88 -358.14) (width 0.25) (layer F.Cu) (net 1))
 (segment (start 55.92 -363.18) (end 55.92 -358.18) (width 0.25) (layer F.Cu) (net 1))
 (via (at 129.54 -353.06) (size 0.8001) (drill 0.8) (layers F.Cu B.Cu) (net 6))
 (segment (start 109.22 -353.06) (end 129.54 -353.06) (width 2) (layer B.Cu) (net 6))
 (segment (start 160.02 -353.06) (end 129.54 -353.06) (width 2) (layer B.Cu) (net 6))
 (via (at 129.54 -350.52) (size 0.8001) (drill 0.8) (layers F.Cu B.Cu) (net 5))
 (segment (start 109.22 -350.52) (end 129.54 -350.52) (width 2) (layer B.Cu) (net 5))
 (segment (start 129.54 -350.52) (end 160.02 -350.52) (width 2) (layer B.Cu) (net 5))
 (segment (start 109.22 -342.9) (end 121.92 -342.9) (width 2) (layer B.Cu) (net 4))
 (segment (start 121.92 -342.9) (end 129.54 -342.9) (width 2) (layer B.Cu) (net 4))
 (via (at 121.92 -342.9) (size 0.8001) (drill 0.8) (layers F.Cu B.Cu) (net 4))
 (segment (start 121.92 -342.9) (end 121.92 -332.74) (width 0.25) (layer F.Cu) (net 4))
 (segment (start 121.92 -332.74) (end 121.92 -332.74) (width 0.25) (layer F.Cu) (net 4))
 (via (at 121.92 -332.74) (size 0.8001) (drill 0.8) (layers F.Cu B.Cu) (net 4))
 (segment (start 121.92 -332.74) (end 66.04 -332.74) (width 2) (layer B.Cu) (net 4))
 (segment (start 66.04 -345.44) (end 50.8 -345.44) (width 2) (layer B.Cu) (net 4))
 (segment (start 109.22 -345.44) (end 114.3 -345.44) (width 2) (layer B.Cu) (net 3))
 (segment (start 114.3 -345.44) (end 129.54 -345.44) (width 2) (layer B.Cu) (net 3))
 (via (at 114.3 -345.44) (size 0.8001) (drill 0.8) (layers F.Cu B.Cu) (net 3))
 (segment (start 114.3 -345.44) (end 114.3 -335.28) (width 0.25) (layer F.Cu) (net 3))
 (segment (start 114.3 -335.28) (end 114.3 -335.28) (width 0.25) (layer F.Cu) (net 3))
 (via (at 114.3 -335.28) (size 0.8001) (drill 0.8) (layers F.Cu B.Cu) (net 3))
 (segment (start 66.04 -347.98) (end 71.12 -347.98) (width 2) (layer B.Cu) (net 3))
 (segment (start 114.3 -335.28) (end 71.12 -335.28) (width 2) (layer B.Cu) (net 3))
 (segment (start 66.04 -347.98) (end 50.8 -347.98) (width 2) (layer B.Cu) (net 3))
 (segment (start 101.6 -347.98) (end 91.44 -347.98) (width 2) (layer B.Cu) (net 8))
 (segment (start 91.44 -347.98) (end 86.36 -347.98) (width 2) (layer B.Cu) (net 8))
 (segment (start 86.36 -347.98) (end 81.28 -347.98) (width 2) (layer B.Cu) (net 8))
 (via (at 86.36 -347.98) (size 0.8001) (drill 0.8) (layers F.Cu B.Cu) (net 8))
 (segment (start 81.28 -342.9) (end 86.36 -342.9) (width 2) (layer B.Cu) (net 9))
 (segment (start 86.36 -342.9) (end 101.6 -342.9) (width 2) (layer B.Cu) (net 9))
 (via (at 86.36 -342.9) (size 0.8001) (drill 0.8) (layers F.Cu B.Cu) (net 9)))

